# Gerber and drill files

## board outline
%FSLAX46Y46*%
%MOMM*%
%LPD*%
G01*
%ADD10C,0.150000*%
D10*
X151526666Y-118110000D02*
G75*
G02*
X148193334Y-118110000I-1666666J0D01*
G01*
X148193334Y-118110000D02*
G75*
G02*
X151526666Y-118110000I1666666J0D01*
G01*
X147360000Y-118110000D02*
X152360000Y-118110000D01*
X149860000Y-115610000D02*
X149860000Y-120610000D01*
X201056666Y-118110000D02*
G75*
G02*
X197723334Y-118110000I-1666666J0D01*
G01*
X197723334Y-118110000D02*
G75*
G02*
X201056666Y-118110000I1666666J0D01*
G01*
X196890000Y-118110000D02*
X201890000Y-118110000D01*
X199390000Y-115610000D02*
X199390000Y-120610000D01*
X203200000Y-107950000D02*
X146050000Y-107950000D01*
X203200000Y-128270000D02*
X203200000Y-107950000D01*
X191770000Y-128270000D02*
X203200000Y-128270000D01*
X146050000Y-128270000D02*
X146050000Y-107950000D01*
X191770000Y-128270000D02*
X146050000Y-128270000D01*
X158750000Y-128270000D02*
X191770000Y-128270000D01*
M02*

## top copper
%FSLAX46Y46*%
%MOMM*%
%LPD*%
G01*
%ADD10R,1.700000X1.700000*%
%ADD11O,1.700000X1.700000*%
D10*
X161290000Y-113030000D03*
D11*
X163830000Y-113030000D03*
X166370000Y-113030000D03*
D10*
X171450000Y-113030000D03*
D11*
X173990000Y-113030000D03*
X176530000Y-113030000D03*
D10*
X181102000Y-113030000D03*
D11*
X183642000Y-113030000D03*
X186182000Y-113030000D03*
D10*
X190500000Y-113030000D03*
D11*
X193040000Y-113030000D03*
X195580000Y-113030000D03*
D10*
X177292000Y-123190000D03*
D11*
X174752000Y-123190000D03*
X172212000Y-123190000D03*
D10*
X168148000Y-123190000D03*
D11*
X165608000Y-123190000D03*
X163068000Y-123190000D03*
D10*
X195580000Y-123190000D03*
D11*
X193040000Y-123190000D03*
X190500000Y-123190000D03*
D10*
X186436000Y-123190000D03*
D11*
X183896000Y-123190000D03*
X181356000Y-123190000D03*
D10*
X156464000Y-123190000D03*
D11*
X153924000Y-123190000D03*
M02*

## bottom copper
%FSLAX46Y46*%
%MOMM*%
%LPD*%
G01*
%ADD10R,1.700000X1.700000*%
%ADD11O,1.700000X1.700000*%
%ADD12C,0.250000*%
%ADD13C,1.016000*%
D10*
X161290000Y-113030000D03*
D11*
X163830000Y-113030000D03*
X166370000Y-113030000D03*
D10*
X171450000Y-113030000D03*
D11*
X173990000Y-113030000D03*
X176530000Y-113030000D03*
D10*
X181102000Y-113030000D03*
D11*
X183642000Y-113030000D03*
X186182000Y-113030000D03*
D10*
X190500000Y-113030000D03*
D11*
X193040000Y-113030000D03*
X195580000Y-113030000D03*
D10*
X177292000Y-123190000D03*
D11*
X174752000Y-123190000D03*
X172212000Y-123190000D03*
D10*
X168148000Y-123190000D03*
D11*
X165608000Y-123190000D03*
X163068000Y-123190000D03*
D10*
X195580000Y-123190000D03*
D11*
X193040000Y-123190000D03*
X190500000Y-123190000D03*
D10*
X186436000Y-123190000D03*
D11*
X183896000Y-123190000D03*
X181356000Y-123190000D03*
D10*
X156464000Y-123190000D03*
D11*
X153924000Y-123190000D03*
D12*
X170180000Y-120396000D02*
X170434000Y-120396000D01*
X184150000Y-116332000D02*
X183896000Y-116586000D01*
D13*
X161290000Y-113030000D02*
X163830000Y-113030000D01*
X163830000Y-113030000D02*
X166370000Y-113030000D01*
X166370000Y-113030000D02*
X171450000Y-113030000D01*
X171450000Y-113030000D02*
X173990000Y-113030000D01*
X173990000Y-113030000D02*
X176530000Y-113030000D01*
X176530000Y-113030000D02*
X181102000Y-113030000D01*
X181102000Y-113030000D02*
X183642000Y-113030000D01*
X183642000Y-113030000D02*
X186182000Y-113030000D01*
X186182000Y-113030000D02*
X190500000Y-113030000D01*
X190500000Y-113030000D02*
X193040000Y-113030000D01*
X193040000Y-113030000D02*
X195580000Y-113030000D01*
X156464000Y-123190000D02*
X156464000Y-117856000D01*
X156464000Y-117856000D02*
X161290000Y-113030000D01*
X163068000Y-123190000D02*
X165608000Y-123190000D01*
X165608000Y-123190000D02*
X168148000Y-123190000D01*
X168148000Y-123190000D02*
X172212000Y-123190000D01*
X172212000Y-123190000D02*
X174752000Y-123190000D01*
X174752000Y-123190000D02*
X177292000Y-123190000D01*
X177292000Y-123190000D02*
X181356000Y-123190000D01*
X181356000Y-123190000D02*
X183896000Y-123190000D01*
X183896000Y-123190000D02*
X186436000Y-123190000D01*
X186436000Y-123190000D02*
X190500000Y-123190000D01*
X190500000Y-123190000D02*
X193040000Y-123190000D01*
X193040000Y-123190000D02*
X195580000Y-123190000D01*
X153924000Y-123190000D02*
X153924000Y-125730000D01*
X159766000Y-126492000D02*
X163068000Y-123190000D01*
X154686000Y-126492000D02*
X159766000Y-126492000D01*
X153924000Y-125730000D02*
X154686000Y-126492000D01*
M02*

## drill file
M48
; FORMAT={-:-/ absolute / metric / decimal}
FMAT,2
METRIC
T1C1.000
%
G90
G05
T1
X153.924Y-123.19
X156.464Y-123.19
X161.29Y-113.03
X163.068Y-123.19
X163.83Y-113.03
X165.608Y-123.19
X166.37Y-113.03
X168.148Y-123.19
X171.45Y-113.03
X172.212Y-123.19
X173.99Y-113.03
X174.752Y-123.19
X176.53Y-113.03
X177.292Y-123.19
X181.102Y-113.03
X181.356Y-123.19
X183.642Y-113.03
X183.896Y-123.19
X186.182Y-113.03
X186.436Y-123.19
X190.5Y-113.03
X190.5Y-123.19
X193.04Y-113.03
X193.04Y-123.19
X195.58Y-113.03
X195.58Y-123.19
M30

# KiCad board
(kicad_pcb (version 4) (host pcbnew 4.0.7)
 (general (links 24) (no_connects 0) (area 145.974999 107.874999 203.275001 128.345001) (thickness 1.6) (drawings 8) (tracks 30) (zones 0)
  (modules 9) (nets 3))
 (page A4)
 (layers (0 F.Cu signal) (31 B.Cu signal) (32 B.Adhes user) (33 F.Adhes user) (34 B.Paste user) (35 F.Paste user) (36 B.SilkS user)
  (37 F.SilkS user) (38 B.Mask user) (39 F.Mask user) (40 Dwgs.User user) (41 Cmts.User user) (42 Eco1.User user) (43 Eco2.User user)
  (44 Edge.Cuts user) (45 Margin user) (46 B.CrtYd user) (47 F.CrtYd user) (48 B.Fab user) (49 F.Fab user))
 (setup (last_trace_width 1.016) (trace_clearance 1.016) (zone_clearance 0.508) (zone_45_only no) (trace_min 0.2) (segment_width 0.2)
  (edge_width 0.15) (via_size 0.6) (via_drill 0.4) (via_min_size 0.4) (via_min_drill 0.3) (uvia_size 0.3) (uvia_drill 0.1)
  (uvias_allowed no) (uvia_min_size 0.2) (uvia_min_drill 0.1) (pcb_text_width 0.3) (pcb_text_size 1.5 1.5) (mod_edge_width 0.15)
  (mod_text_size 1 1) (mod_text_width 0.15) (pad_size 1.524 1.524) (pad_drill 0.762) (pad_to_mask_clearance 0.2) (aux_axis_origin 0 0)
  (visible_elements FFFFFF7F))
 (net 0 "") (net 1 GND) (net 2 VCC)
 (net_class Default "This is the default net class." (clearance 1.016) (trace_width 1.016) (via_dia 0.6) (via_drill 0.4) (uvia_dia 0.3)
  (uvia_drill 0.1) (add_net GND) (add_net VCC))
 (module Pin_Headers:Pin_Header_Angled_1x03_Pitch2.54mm (layer F.Cu) (at 161.29 113.03 90)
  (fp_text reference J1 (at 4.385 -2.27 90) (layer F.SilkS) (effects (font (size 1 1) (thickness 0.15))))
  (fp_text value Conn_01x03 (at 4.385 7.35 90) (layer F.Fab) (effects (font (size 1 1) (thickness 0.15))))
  (pad 1 thru_hole rect (at 0 0 90) (size 1.7 1.7) (drill 1) (layers *.Cu *.Mask) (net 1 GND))
  (pad 2 thru_hole oval (at 0 2.54 90) (size 1.7 1.7) (drill 1) (layers *.Cu *.Mask) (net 1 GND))
  (pad 3 thru_hole oval (at 0 5.08 90) (size 1.7 1.7) (drill 1) (layers *.Cu *.Mask) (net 1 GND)))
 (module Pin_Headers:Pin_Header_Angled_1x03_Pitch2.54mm (layer F.Cu) (at 171.45 113.03 90)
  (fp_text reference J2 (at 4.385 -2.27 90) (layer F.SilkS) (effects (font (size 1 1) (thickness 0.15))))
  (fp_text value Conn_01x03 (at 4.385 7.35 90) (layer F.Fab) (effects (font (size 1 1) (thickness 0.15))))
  (pad 1 thru_hole rect (at 0 0 90) (size 1.7 1.7) (drill 1) (layers *.Cu *.Mask) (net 1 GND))
  (pad 2 thru_hole oval (at 0 2.54 90) (size 1.7 1.7) (drill 1) (layers *.Cu *.Mask) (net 1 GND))
  (pad 3 thru_hole oval (at 0 5.08 90) (size 1.7 1.7) (drill 1) (layers *.Cu *.Mask) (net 1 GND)))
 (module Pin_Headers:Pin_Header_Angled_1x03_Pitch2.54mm (layer F.Cu) (at 181.102 113.03 90)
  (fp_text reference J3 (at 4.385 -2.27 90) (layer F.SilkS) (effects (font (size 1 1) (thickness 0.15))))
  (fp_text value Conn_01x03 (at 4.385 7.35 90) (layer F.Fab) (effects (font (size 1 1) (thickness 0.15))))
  (pad 1 thru_hole rect (at 0 0 90) (size 1.7 1.7) (drill 1) (layers *.Cu *.Mask) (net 1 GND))
  (pad 2 thru_hole oval (at 0 2.54 90) (size 1.7 1.7) (drill 1) (layers *.Cu *.Mask) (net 1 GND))
  (pad 3 thru_hole oval (at 0 5.08 90) (size 1.7 1.7) (drill 1) (layers *.Cu *.Mask) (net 1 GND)))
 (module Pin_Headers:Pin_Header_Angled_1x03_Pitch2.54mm (layer F.Cu) (at 190.5 113.03 90)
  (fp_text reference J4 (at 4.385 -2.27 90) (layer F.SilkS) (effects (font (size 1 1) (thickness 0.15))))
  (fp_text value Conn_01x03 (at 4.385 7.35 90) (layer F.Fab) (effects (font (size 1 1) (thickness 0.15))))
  (pad 1 thru_hole rect (at 0 0 90) (size 1.7 1.7) (drill 1) (layers *.Cu *.Mask) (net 1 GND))
  (pad 2 thru_hole oval (at 0 2.54 90) (size 1.7 1.7) (drill 1) (layers *.Cu *.Mask) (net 1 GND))
  (pad 3 thru_hole oval (at 0 5.08 90) (size 1.7 1.7) (drill 1) (layers *.Cu *.Mask) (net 1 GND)))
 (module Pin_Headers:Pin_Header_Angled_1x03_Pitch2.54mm (layer F.Cu) (at 177.292 123.19 270)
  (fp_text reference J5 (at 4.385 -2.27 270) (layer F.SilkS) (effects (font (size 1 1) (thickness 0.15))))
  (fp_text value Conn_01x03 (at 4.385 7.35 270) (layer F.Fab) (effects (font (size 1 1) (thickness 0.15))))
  (pad 1 thru_hole rect (at 0 0 270) (size 1.7 1.7) (drill 1) (layers *.Cu *.Mask) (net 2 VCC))
  (pad 2 thru_hole oval (at 0 2.54 270) (size 1.7 1.7) (drill 1) (layers *.Cu *.Mask) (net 2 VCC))
  (pad 3 thru_hole oval (at 0 5.08 270) (size 1.7 1.7) (drill 1) (layers *.Cu *.Mask) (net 2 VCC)))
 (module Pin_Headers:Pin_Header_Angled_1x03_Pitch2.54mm (layer F.Cu) (at 168.148 123.19 270)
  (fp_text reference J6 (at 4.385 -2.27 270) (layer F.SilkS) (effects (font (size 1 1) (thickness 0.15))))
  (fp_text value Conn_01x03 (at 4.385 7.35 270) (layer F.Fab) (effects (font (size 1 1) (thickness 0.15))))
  (pad 1 thru_hole rect (at 0 0 270) (size 1.7 1.7) (drill 1) (layers *.Cu *.Mask) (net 2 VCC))
  (pad 2 thru_hole oval (at 0 2.54 270) (size 1.7 1.7) (drill 1) (layers *.Cu *.Mask) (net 2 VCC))
  (pad 3 thru_hole oval (at 0 5.08 270) (size 1.7 1.7) (drill 1) (layers *.Cu *.Mask) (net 2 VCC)))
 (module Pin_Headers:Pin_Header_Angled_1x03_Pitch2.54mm (layer F.Cu) (at 195.58 123.19 270)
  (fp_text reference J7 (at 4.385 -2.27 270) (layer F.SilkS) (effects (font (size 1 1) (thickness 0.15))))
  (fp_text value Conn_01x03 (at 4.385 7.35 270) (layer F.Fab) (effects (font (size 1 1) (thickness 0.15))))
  (pad 1 thru_hole rect (at 0 0 270) (size 1.7 1.7) (drill 1) (layers *.Cu *.Mask) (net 2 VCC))
  (pad 2 thru_hole oval (at 0 2.54 270) (size 1.7 1.7) (drill 1) (layers *.Cu *.Mask) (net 2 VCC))
  (pad 3 thru_hole oval (at 0 5.08 270) (size 1.7 1.7) (drill 1) (layers *.Cu *.Mask) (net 2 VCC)))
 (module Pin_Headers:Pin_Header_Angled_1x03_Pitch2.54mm (layer F.Cu) (at 186.436 123.19 270)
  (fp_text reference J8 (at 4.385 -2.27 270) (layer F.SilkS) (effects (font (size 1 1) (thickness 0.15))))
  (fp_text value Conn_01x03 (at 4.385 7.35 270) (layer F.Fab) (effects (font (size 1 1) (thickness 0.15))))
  (pad 1 thru_hole rect (at 0 0 270) (size 1.7 1.7) (drill 1) (layers *.Cu *.Mask) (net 2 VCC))
  (pad 2 thru_hole oval (at 0 2.54 270) (size 1.7 1.7) (drill 1) (layers *.Cu *.Mask) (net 2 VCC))
  (pad 3 thru_hole oval (at 0 5.08 270) (size 1.7 1.7) (drill 1) (layers *.Cu *.Mask) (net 2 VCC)))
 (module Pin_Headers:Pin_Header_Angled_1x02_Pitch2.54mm (layer F.Cu) (at 156.464 123.19 270)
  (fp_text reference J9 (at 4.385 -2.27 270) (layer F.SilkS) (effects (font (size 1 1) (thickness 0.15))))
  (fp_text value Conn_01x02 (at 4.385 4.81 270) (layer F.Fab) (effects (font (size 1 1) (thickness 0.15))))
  (pad 1 thru_hole rect (at 0 0 270) (size 1.7 1.7) (drill 1) (layers *.Cu *.Mask) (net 1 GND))
  (pad 2 thru_hole oval (at 0 2.54 270) (size 1.7 1.7) (drill 1) (layers *.Cu *.Mask) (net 2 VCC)))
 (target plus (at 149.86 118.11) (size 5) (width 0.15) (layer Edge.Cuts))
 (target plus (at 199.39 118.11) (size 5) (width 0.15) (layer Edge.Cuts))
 (gr_line (start 203.2 107.95) (end 146.05 107.95) (angle 90) (layer Edge.Cuts) (width 0.15))
 (gr_line (start 203.2 128.27) (end 203.2 107.95) (angle 90) (layer Edge.Cuts) (width 0.15))
 (gr_line (start 191.77 128.27) (end 203.2 128.27) (angle 90) (layer Edge.Cuts) (width 0.15))
 (gr_line (start 146.05 128.27) (end 146.05 107.95) (angle 90) (layer Edge.Cuts) (width 0.15))
 (gr_line (start 191.77 128.27) (end 146.05 128.27) (angle 90) (layer Edge.Cuts) (width 0.15))
 (gr_line (start 158.75 128.27) (end 191.77 128.27) (angle 90) (layer Edge.Cuts) (width 0.15))
 (segment (start 170.18 120.396) (end 170.434 120.396) (width 0.25) (layer B.Cu) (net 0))
 (segment (start 184.15 116.332) (end 183.896 116.586) (width 0.25) (layer B.Cu) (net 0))
 (segment (start 161.29 113.03) (end 163.83 113.03) (width 1.016) (layer B.Cu) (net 1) (status C00000))
 (segment (start 163.83 113.03) (end 166.37 113.03) (width 1.016) (layer B.Cu) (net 1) (status C00000))
 (segment (start 166.37 113.03) (end 171.45 113.03) (width 1.016) (layer B.Cu) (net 1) (status C00000))
 (segment (start 171.45 113.03) (end 173.99 113.03) (width 1.016) (layer B.Cu) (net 1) (status C00000))
 (segment (start 173.99 113.03) (end 176.53 113.03) (width 1.016) (layer B.Cu) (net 1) (status C00000))
 (segment (start 176.53 113.03) (end 181.102 113.03) (width 1.016) (layer B.Cu) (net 1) (status C00000))
 (segment (start 181.102 113.03) (end 183.642 113.03) (width 1.016) (layer B.Cu) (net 1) (status C00000))
 (segment (start 183.642 113.03) (end 186.182 113.03) (width 1.016) (layer B.Cu) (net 1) (status C00000))
 (segment (start 186.182 113.03) (end 190.5 113.03) (width 1.016) (layer B.Cu) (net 1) (status C00000))
 (segment (start 190.5 113.03) (end 193.04 113.03) (width 1.016) (layer B.Cu) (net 1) (status C00000))
 (segment (start 193.04 113.03) (end 195.58 113.03) (width 1.016) (layer B.Cu) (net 1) (status C00000))
 (segment (start 156.464 123.19) (end 156.464 117.856) (width 1.016) (layer B.Cu) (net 1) (status 400000))
 (segment (start 156.464 117.856) (end 161.29 113.03) (width 1.016) (layer B.Cu) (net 1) (status 800000))
 (segment (start 163.068 123.19) (end 165.608 123.19) (width 1.016) (layer B.Cu) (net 2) (status C00000))
 (segment (start 165.608 123.19) (end 168.148 123.19) (width 1.016) (layer B.Cu) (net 2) (status C00000))
 (segment (start 168.148 123.19) (end 172.212 123.19) (width 1.016) (layer B.Cu) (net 2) (status C00000))
 (segment (start 172.212 123.19) (end 174.752 123.19) (width 1.016) (layer B.Cu) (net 2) (status C00000))
 (segment (start 174.752 123.19) (end 177.292 123.19) (width 1.016) (layer B.Cu) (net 2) (status C00000))
 (segment (start 177.292 123.19) (end 181.356 123.19) (width 1.016) (layer B.Cu) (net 2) (status C00000))
 (segment (start 181.356 123.19) (end 183.896 123.19) (width 1.016) (layer B.Cu) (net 2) (status C00000))
 (segment (start 183.896 123.19) (end 186.436 123.19) (width 1.016) (layer B.Cu) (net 2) (status C00000))
 (segment (start 186.436 123.19) (end 190.5 123.19) (width 1.016) (layer B.Cu) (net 2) (status C00000))
 (segment (start 190.5 123.19) (end 193.04 123.19) (width 1.016) (layer B.Cu) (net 2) (status C00000))
 (segment (start 193.04 123.19) (end 195.58 123.19) (width 1.016) (layer B.Cu) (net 2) (status C00000))
 (segment (start 153.924 123.19) (end 153.924 125.73) (width 1.016) (layer B.Cu) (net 2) (status 400000))
 (segment (start 159.766 126.492) (end 163.068 123.19) (width 1.016) (layer B.Cu) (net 2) (status 800000))
 (segment (start 154.686 126.492) (end 159.766 126.492) (width 1.016) (layer B.Cu) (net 2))
 (segment (start 153.924 125.73) (end 154.686 126.492) (width 1.016) (layer B.Cu) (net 2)))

